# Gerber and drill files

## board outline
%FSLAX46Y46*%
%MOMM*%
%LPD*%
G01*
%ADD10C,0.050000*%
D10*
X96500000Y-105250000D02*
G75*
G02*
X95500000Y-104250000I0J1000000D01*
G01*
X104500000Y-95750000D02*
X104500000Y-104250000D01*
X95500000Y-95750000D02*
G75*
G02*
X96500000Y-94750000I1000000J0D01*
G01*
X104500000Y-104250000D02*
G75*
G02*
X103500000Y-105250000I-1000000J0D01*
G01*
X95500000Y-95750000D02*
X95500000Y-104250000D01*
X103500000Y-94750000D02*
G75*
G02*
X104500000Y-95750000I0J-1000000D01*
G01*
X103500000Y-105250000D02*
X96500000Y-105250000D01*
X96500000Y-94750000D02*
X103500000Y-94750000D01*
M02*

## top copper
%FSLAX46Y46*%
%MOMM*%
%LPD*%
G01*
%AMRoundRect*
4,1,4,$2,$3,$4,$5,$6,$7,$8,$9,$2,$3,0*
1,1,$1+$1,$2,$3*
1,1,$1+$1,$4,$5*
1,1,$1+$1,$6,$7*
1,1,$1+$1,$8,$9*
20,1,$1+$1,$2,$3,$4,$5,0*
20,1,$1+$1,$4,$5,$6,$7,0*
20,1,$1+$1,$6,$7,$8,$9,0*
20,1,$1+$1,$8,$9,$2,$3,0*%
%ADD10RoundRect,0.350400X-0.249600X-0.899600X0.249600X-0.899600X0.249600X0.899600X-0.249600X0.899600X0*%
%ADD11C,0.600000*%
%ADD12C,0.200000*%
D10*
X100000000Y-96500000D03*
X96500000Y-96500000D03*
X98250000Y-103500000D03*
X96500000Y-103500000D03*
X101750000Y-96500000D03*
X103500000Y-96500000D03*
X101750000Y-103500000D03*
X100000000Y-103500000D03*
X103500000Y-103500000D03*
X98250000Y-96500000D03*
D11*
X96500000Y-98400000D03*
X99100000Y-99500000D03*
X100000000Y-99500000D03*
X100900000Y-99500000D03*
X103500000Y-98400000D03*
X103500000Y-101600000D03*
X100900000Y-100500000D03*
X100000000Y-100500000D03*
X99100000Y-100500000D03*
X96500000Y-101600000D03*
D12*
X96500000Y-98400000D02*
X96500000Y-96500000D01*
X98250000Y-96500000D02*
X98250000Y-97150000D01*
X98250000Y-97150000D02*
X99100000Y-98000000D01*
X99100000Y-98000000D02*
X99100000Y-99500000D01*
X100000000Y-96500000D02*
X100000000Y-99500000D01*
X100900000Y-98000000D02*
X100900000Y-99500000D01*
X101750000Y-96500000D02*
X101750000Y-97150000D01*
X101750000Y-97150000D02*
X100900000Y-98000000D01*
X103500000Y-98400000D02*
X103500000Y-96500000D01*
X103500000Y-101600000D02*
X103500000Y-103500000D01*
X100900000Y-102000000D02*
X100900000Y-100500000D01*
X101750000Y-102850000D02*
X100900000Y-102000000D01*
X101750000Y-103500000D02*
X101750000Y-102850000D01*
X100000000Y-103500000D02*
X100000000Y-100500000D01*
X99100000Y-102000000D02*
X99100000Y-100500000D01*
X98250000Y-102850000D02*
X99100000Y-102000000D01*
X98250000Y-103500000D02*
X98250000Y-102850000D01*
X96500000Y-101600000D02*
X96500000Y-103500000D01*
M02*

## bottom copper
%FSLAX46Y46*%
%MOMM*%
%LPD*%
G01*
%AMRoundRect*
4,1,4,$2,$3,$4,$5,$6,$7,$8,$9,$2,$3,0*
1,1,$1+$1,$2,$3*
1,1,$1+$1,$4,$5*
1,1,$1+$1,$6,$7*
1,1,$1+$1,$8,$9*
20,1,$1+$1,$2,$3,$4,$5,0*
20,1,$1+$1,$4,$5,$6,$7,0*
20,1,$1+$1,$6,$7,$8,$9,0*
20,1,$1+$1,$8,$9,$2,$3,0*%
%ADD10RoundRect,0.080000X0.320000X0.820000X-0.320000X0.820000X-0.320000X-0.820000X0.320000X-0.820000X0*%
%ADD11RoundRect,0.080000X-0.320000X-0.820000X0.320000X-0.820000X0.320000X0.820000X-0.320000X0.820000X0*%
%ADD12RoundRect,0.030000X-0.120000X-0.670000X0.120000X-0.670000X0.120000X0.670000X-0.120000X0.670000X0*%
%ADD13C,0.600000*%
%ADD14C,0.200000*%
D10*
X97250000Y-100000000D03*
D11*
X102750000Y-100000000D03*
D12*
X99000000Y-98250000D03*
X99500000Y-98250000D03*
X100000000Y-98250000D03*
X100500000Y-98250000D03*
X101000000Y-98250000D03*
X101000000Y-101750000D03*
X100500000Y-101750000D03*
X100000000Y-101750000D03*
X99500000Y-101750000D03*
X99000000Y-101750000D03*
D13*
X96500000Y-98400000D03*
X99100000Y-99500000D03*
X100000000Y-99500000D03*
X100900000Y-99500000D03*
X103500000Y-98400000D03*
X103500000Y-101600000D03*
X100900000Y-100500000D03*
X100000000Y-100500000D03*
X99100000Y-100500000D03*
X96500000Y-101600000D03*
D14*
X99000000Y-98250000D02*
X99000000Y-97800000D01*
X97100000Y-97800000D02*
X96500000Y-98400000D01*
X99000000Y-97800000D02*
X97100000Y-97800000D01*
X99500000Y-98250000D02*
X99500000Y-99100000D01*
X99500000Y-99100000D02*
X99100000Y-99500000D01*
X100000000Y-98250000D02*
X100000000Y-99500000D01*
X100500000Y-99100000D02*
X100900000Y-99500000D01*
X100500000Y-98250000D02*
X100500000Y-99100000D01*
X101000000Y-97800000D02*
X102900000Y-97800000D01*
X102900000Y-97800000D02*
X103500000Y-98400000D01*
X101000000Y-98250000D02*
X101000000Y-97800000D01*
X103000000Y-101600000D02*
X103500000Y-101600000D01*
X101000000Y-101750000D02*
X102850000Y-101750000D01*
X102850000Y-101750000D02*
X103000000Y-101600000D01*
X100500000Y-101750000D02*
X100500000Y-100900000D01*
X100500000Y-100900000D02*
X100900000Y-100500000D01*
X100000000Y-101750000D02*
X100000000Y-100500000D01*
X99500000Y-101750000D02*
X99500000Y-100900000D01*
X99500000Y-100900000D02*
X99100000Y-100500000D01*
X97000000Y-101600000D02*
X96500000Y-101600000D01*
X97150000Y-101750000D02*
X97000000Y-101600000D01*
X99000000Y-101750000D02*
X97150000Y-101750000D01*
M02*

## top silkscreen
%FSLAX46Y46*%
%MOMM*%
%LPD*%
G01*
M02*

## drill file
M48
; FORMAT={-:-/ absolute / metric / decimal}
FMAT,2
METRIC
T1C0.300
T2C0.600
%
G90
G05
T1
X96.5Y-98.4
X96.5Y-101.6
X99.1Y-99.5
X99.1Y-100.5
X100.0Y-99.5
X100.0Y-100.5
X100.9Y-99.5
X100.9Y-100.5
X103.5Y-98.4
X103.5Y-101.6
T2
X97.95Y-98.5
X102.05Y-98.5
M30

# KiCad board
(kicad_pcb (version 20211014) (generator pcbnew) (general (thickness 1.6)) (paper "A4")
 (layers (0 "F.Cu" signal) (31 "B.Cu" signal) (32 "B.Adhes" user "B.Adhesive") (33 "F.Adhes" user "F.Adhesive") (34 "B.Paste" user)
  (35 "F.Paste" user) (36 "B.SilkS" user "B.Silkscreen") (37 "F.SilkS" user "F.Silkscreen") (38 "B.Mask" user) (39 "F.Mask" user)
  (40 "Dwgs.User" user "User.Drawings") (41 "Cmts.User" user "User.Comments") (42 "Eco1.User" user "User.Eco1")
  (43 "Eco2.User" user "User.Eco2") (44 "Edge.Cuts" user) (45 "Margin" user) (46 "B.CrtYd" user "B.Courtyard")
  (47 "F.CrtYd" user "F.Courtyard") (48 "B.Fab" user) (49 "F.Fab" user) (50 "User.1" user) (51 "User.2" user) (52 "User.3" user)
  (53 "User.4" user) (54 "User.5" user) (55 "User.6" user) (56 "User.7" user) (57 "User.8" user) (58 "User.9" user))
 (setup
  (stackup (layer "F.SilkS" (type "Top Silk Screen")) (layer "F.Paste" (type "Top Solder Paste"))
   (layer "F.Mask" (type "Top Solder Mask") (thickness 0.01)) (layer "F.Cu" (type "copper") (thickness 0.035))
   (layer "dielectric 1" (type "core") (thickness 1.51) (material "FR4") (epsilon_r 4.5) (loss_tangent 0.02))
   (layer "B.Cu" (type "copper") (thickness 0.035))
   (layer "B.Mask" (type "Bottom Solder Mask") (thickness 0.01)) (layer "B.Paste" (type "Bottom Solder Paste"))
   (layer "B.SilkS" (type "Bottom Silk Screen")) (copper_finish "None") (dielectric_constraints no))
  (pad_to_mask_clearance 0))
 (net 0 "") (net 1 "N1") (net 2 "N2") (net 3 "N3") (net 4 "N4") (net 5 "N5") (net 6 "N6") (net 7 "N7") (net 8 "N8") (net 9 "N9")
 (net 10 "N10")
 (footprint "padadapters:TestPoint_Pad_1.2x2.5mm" (layer "F.Cu") (at 100 96.5)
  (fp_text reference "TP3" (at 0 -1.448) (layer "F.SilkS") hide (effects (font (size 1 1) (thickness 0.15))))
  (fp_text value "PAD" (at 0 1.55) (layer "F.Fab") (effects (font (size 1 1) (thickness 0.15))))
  (pad "1" smd roundrect (at 0 0) (size 1.2 2.5) (layers "F.Cu" "F.Mask") (roundrect_rratio 0.292) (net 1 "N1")))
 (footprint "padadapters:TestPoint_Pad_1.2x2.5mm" (layer "F.Cu") (at 96.5 96.5)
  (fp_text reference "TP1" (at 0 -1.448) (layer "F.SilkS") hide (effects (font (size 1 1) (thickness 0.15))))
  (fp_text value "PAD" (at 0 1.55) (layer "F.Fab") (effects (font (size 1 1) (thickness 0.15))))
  (pad "1" smd roundrect (at 0 0) (size 1.2 2.5) (layers "F.Cu" "F.Mask") (roundrect_rratio 0.292) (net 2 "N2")))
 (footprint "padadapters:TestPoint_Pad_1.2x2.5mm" (layer "F.Cu") (at 98.25 103.5)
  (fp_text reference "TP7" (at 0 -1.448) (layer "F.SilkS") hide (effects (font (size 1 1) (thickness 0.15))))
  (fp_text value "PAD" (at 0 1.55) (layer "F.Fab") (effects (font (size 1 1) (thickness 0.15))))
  (pad "1" smd roundrect (at 0 0) (size 1.2 2.5) (layers "F.Cu" "F.Mask") (roundrect_rratio 0.292) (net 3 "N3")))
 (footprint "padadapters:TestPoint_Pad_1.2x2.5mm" (layer "F.Cu") (at 96.5 103.5)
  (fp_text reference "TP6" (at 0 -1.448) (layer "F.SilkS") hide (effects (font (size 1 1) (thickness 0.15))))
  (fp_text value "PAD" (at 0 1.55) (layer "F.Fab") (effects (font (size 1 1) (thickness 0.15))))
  (pad "1" smd roundrect (at 0 0) (size 1.2 2.5) (layers "F.Cu" "F.Mask") (roundrect_rratio 0.292) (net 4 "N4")))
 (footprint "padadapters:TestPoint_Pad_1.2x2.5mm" (layer "F.Cu") (at 101.75 96.5)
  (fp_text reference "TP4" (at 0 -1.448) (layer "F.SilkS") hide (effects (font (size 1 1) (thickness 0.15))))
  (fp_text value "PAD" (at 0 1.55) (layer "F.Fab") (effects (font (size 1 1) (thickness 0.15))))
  (pad "1" smd roundrect (at 0 0) (size 1.2 2.5) (layers "F.Cu" "F.Mask") (roundrect_rratio 0.292) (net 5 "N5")))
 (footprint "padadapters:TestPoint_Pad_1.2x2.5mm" (layer "F.Cu") (at 103.5 96.5)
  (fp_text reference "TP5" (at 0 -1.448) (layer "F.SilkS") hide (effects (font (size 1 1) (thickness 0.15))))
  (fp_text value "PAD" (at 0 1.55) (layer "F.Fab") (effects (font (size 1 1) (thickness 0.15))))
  (pad "1" smd roundrect (at 0 0) (size 1.2 2.5) (layers "F.Cu" "F.Mask") (roundrect_rratio 0.292) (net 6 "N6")))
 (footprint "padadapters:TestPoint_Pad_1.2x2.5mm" (layer "F.Cu") (at 101.75 103.5)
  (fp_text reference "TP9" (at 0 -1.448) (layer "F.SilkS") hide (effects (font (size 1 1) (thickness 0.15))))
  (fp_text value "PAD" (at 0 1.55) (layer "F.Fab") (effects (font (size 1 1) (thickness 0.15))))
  (pad "1" smd roundrect (at 0 0) (size 1.2 2.5) (layers "F.Cu" "F.Mask") (roundrect_rratio 0.292) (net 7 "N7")))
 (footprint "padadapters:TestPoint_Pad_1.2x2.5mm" (layer "F.Cu") (at 100 103.5)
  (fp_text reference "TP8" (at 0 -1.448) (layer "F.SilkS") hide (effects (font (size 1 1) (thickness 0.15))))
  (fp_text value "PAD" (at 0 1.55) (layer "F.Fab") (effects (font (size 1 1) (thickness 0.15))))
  (pad "1" smd roundrect (at 0 0) (size 1.2 2.5) (layers "F.Cu" "F.Mask") (roundrect_rratio 0.292) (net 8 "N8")))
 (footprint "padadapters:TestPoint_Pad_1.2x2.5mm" (layer "F.Cu") (at 103.5 103.5)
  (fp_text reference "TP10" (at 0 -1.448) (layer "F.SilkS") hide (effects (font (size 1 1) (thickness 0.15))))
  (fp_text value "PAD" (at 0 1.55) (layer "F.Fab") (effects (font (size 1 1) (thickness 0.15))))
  (pad "1" smd roundrect (at 0 0) (size 1.2 2.5) (layers "F.Cu" "F.Mask") (roundrect_rratio 0.292) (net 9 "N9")))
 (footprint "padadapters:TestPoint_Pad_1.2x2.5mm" (layer "F.Cu") (at 98.25 96.5)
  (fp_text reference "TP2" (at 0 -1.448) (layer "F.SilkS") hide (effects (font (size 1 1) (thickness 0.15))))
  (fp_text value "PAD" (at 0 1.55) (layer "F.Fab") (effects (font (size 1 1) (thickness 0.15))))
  (pad "1" smd roundrect (at 0 0) (size 1.2 2.5) (layers "F.Cu" "F.Mask") (roundrect_rratio 0.292) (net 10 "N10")))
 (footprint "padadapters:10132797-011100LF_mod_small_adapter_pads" (layer "B.Cu") (at 100 100 180)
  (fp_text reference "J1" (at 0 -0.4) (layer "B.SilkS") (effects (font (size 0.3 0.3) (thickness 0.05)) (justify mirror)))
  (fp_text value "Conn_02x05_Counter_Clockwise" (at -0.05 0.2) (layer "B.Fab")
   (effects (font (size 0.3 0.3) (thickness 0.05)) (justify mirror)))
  (pad "" np_thru_hole circle (at -2.05 1.5 180) (size 0.6 0.6) (drill 0.6) (layers *.Cu *.Mask) (solder_mask_margin -0.001))
  (pad "" smd roundrect (at 2.75 0 180) (size 0.8 1.8) (layers "B.Cu" "B.Paste" "B.Mask") (roundrect_rratio 0.1))
  (pad "" np_thru_hole circle (at 2.05 1.5 180) (size 0.6 0.6) (drill 0.6) (layers *.Cu *.Mask) (solder_mask_margin -0.001))
  (pad "" smd roundrect (at -2.75 0) (size 0.8 1.8) (layers "B.Cu" "B.Paste" "B.Mask") (roundrect_rratio 0.1))
  (pad "1" smd roundrect (at 1 1.75) (size 0.3 1.4) (layers "B.Cu" "B.Paste" "B.Mask") (roundrect_rratio 0.1) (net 2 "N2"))
  (pad "2" smd roundrect (at 0.5 1.75) (size 0.3 1.4) (layers "B.Cu" "B.Paste" "B.Mask") (roundrect_rratio 0.1) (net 10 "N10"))
  (pad "3" smd roundrect (at 0 1.75) (size 0.3 1.4) (layers "B.Cu" "B.Paste" "B.Mask") (roundrect_rratio 0.1) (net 1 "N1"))
  (pad "4" smd roundrect (at -0.5 1.75) (size 0.3 1.4) (layers "B.Cu" "B.Paste" "B.Mask") (roundrect_rratio 0.1) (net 5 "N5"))
  (pad "5" smd roundrect (at -1 1.75) (size 0.3 1.4) (layers "B.Cu" "B.Paste" "B.Mask") (roundrect_rratio 0.1) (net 6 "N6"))
  (pad "6" smd roundrect (at -1 -1.75) (size 0.3 1.4) (layers "B.Cu" "B.Paste" "B.Mask") (roundrect_rratio 0.1) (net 9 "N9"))
  (pad "7" smd roundrect (at -0.5 -1.75) (size 0.3 1.4) (layers "B.Cu" "B.Paste" "B.Mask") (roundrect_rratio 0.1) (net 7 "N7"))
  (pad "8" smd roundrect (at 0 -1.75) (size 0.3 1.4) (layers "B.Cu" "B.Paste" "B.Mask") (roundrect_rratio 0.1) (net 8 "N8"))
  (pad "9" smd roundrect (at 0.5 -1.75) (size 0.3 1.4) (layers "B.Cu" "B.Paste" "B.Mask") (roundrect_rratio 0.1) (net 3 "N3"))
  (pad "10" smd roundrect (at 1 -1.75) (size 0.3 1.4) (layers "B.Cu" "B.Paste" "B.Mask") (roundrect_rratio 0.1) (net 4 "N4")))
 (gr_arc (start 96.5 105.25) (mid 95.792893 104.957107) (end 95.5 104.25) (layer "Edge.Cuts") (width 0.05))
 (gr_line (start 104.5 95.75) (end 104.5 104.25) (layer "Edge.Cuts") (width 0.05))
 (gr_arc (start 95.5 95.75) (mid 95.792893 95.042893) (end 96.5 94.75) (layer "Edge.Cuts") (width 0.05))
 (gr_arc (start 104.5 104.25) (mid 104.207107 104.957107) (end 103.5 105.25) (layer "Edge.Cuts") (width 0.05))
 (gr_line (start 95.5 95.75) (end 95.5 104.25) (layer "Edge.Cuts") (width 0.05))
 (gr_arc (start 103.5 94.75) (mid 104.207107 95.042893) (end 104.5 95.75) (layer "Edge.Cuts") (width 0.05))
 (gr_line (start 103.5 105.25) (end 96.5 105.25) (layer "Edge.Cuts") (width 0.05))
 (gr_line (start 96.5 94.75) (end 103.5 94.75) (layer "Edge.Cuts") (width 0.05))
 (segment (start 96.5 98.4) (end 96.5 96.5) (width 0.2) (layer "F.Cu") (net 2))
 (via (at 96.5 98.4) (size 0.6) (drill 0.3) (layers "F.Cu" "B.Cu") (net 2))
 (segment (start 99 98.25) (end 99 97.8) (width 0.2) (layer "B.Cu") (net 2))
 (segment (start 97.1 97.8) (end 96.5 98.4) (width 0.2) (layer "B.Cu") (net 2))
 (segment (start 99 97.8) (end 97.1 97.8) (width 0.2) (layer "B.Cu") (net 2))
 (segment (start 98.25 96.5) (end 98.25 97.15) (width 0.2) (layer "F.Cu") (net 10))
 (segment (start 98.25 97.15) (end 99.1 98) (width 0.2) (layer "F.Cu") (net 10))
 (segment (start 99.1 98) (end 99.1 99.5) (width 0.2) (layer "F.Cu") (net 10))
 (via (at 99.1 99.5) (size 0.6) (drill 0.3) (layers "F.Cu" "B.Cu") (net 10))
 (segment (start 99.5 98.25) (end 99.5 99.1) (width 0.2) (layer "B.Cu") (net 10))
 (segment (start 99.5 99.1) (end 99.1 99.5) (width 0.2) (layer "B.Cu") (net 10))
 (segment (start 100 96.5) (end 100 99.5) (width 0.2) (layer "F.Cu") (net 1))
 (via (at 100 99.5) (size 0.6) (drill 0.3) (layers "F.Cu" "B.Cu") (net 1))
 (segment (start 100 98.25) (end 100 99.5) (width 0.2) (layer "B.Cu") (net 1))
 (segment (start 100.9 98) (end 100.9 99.5) (width 0.2) (layer "F.Cu") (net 5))
 (segment (start 101.75 96.5) (end 101.75 97.15) (width 0.2) (layer "F.Cu") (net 5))
 (segment (start 101.75 97.15) (end 100.9 98) (width 0.2) (layer "F.Cu") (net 5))
 (via (at 100.9 99.5) (size 0.6) (drill 0.3) (layers "F.Cu" "B.Cu") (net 5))
 (segment (start 100.5 99.1) (end 100.9 99.5) (width 0.2) (layer "B.Cu") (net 5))
 (segment (start 100.5 98.25) (end 100.5 99.1) (width 0.2) (layer "B.Cu") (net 5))
 (segment (start 103.5 98.4) (end 103.5 96.5) (width 0.2) (layer "F.Cu") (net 6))
 (via (at 103.5 98.4) (size 0.6) (drill 0.3) (layers "F.Cu" "B.Cu") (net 6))
 (segment (start 101 97.8) (end 102.9 97.8) (width 0.2) (layer "B.Cu") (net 6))
 (segment (start 102.9 97.8) (end 103.5 98.4) (width 0.2) (layer "B.Cu") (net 6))
 (segment (start 101 98.25) (end 101 97.8) (width 0.2) (layer "B.Cu") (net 6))
 (segment (start 103.5 101.6) (end 103.5 103.5) (width 0.2) (layer "F.Cu") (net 9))
 (via (at 103.5 101.6) (size 0.6) (drill 0.3) (layers "F.Cu" "B.Cu") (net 9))
 (segment (start 103 101.6) (end 103.5 101.6) (width 0.2) (layer "B.Cu") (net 9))
 (segment (start 101 101.75) (end 102.85 101.75) (width 0.2) (layer "B.Cu") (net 9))
 (segment (start 102.85 101.75) (end 103 101.6) (width 0.2) (layer "B.Cu") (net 9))
 (segment (start 100.9 102) (end 100.9 100.5) (width 0.2) (layer "F.Cu") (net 7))
 (segment (start 101.75 102.85) (end 100.9 102) (width 0.2) (layer "F.Cu") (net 7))
 (segment (start 101.75 103.5) (end 101.75 102.85) (width 0.2) (layer "F.Cu") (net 7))
 (via (at 100.9 100.5) (size 0.6) (drill 0.3) (layers "F.Cu" "B.Cu") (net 7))
 (segment (start 100.5 101.75) (end 100.5 100.9) (width 0.2) (layer "B.Cu") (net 7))
 (segment (start 100.5 100.9) (end 100.9 100.5) (width 0.2) (layer "B.Cu") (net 7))
 (segment (start 100 103.5) (end 100 100.5) (width 0.2) (layer "F.Cu") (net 8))
 (via (at 100 100.5) (size 0.6) (drill 0.3) (layers "F.Cu" "B.Cu") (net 8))
 (segment (start 100 101.75) (end 100 100.5) (width 0.2) (layer "B.Cu") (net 8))
 (segment (start 99.1 102) (end 99.1 100.5) (width 0.2) (layer "F.Cu") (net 3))
 (segment (start 98.25 102.85) (end 99.1 102) (width 0.2) (layer "F.Cu") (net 3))
 (segment (start 98.25 103.5) (end 98.25 102.85) (width 0.2) (layer "F.Cu") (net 3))
 (via (at 99.1 100.5) (size 0.6) (drill 0.3) (layers "F.Cu" "B.Cu") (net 3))
 (segment (start 99.5 101.75) (end 99.5 100.9) (width 0.2) (layer "B.Cu") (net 3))
 (segment (start 99.5 100.9) (end 99.1 100.5) (width 0.2) (layer "B.Cu") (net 3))
 (segment (start 96.5 101.6) (end 96.5 103.5) (width 0.2) (layer "F.Cu") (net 4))
 (via (at 96.5 101.6) (size 0.6) (drill 0.3) (layers "F.Cu" "B.Cu") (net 4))
 (segment (start 97 101.6) (end 96.5 101.6) (width 0.2) (layer "B.Cu") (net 4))
 (segment (start 97.15 101.75) (end 97 101.6) (width 0.2) (layer "B.Cu") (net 4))
 (segment (start 99 101.75) (end 97.15 101.75) (width 0.2) (layer "B.Cu") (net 4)))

